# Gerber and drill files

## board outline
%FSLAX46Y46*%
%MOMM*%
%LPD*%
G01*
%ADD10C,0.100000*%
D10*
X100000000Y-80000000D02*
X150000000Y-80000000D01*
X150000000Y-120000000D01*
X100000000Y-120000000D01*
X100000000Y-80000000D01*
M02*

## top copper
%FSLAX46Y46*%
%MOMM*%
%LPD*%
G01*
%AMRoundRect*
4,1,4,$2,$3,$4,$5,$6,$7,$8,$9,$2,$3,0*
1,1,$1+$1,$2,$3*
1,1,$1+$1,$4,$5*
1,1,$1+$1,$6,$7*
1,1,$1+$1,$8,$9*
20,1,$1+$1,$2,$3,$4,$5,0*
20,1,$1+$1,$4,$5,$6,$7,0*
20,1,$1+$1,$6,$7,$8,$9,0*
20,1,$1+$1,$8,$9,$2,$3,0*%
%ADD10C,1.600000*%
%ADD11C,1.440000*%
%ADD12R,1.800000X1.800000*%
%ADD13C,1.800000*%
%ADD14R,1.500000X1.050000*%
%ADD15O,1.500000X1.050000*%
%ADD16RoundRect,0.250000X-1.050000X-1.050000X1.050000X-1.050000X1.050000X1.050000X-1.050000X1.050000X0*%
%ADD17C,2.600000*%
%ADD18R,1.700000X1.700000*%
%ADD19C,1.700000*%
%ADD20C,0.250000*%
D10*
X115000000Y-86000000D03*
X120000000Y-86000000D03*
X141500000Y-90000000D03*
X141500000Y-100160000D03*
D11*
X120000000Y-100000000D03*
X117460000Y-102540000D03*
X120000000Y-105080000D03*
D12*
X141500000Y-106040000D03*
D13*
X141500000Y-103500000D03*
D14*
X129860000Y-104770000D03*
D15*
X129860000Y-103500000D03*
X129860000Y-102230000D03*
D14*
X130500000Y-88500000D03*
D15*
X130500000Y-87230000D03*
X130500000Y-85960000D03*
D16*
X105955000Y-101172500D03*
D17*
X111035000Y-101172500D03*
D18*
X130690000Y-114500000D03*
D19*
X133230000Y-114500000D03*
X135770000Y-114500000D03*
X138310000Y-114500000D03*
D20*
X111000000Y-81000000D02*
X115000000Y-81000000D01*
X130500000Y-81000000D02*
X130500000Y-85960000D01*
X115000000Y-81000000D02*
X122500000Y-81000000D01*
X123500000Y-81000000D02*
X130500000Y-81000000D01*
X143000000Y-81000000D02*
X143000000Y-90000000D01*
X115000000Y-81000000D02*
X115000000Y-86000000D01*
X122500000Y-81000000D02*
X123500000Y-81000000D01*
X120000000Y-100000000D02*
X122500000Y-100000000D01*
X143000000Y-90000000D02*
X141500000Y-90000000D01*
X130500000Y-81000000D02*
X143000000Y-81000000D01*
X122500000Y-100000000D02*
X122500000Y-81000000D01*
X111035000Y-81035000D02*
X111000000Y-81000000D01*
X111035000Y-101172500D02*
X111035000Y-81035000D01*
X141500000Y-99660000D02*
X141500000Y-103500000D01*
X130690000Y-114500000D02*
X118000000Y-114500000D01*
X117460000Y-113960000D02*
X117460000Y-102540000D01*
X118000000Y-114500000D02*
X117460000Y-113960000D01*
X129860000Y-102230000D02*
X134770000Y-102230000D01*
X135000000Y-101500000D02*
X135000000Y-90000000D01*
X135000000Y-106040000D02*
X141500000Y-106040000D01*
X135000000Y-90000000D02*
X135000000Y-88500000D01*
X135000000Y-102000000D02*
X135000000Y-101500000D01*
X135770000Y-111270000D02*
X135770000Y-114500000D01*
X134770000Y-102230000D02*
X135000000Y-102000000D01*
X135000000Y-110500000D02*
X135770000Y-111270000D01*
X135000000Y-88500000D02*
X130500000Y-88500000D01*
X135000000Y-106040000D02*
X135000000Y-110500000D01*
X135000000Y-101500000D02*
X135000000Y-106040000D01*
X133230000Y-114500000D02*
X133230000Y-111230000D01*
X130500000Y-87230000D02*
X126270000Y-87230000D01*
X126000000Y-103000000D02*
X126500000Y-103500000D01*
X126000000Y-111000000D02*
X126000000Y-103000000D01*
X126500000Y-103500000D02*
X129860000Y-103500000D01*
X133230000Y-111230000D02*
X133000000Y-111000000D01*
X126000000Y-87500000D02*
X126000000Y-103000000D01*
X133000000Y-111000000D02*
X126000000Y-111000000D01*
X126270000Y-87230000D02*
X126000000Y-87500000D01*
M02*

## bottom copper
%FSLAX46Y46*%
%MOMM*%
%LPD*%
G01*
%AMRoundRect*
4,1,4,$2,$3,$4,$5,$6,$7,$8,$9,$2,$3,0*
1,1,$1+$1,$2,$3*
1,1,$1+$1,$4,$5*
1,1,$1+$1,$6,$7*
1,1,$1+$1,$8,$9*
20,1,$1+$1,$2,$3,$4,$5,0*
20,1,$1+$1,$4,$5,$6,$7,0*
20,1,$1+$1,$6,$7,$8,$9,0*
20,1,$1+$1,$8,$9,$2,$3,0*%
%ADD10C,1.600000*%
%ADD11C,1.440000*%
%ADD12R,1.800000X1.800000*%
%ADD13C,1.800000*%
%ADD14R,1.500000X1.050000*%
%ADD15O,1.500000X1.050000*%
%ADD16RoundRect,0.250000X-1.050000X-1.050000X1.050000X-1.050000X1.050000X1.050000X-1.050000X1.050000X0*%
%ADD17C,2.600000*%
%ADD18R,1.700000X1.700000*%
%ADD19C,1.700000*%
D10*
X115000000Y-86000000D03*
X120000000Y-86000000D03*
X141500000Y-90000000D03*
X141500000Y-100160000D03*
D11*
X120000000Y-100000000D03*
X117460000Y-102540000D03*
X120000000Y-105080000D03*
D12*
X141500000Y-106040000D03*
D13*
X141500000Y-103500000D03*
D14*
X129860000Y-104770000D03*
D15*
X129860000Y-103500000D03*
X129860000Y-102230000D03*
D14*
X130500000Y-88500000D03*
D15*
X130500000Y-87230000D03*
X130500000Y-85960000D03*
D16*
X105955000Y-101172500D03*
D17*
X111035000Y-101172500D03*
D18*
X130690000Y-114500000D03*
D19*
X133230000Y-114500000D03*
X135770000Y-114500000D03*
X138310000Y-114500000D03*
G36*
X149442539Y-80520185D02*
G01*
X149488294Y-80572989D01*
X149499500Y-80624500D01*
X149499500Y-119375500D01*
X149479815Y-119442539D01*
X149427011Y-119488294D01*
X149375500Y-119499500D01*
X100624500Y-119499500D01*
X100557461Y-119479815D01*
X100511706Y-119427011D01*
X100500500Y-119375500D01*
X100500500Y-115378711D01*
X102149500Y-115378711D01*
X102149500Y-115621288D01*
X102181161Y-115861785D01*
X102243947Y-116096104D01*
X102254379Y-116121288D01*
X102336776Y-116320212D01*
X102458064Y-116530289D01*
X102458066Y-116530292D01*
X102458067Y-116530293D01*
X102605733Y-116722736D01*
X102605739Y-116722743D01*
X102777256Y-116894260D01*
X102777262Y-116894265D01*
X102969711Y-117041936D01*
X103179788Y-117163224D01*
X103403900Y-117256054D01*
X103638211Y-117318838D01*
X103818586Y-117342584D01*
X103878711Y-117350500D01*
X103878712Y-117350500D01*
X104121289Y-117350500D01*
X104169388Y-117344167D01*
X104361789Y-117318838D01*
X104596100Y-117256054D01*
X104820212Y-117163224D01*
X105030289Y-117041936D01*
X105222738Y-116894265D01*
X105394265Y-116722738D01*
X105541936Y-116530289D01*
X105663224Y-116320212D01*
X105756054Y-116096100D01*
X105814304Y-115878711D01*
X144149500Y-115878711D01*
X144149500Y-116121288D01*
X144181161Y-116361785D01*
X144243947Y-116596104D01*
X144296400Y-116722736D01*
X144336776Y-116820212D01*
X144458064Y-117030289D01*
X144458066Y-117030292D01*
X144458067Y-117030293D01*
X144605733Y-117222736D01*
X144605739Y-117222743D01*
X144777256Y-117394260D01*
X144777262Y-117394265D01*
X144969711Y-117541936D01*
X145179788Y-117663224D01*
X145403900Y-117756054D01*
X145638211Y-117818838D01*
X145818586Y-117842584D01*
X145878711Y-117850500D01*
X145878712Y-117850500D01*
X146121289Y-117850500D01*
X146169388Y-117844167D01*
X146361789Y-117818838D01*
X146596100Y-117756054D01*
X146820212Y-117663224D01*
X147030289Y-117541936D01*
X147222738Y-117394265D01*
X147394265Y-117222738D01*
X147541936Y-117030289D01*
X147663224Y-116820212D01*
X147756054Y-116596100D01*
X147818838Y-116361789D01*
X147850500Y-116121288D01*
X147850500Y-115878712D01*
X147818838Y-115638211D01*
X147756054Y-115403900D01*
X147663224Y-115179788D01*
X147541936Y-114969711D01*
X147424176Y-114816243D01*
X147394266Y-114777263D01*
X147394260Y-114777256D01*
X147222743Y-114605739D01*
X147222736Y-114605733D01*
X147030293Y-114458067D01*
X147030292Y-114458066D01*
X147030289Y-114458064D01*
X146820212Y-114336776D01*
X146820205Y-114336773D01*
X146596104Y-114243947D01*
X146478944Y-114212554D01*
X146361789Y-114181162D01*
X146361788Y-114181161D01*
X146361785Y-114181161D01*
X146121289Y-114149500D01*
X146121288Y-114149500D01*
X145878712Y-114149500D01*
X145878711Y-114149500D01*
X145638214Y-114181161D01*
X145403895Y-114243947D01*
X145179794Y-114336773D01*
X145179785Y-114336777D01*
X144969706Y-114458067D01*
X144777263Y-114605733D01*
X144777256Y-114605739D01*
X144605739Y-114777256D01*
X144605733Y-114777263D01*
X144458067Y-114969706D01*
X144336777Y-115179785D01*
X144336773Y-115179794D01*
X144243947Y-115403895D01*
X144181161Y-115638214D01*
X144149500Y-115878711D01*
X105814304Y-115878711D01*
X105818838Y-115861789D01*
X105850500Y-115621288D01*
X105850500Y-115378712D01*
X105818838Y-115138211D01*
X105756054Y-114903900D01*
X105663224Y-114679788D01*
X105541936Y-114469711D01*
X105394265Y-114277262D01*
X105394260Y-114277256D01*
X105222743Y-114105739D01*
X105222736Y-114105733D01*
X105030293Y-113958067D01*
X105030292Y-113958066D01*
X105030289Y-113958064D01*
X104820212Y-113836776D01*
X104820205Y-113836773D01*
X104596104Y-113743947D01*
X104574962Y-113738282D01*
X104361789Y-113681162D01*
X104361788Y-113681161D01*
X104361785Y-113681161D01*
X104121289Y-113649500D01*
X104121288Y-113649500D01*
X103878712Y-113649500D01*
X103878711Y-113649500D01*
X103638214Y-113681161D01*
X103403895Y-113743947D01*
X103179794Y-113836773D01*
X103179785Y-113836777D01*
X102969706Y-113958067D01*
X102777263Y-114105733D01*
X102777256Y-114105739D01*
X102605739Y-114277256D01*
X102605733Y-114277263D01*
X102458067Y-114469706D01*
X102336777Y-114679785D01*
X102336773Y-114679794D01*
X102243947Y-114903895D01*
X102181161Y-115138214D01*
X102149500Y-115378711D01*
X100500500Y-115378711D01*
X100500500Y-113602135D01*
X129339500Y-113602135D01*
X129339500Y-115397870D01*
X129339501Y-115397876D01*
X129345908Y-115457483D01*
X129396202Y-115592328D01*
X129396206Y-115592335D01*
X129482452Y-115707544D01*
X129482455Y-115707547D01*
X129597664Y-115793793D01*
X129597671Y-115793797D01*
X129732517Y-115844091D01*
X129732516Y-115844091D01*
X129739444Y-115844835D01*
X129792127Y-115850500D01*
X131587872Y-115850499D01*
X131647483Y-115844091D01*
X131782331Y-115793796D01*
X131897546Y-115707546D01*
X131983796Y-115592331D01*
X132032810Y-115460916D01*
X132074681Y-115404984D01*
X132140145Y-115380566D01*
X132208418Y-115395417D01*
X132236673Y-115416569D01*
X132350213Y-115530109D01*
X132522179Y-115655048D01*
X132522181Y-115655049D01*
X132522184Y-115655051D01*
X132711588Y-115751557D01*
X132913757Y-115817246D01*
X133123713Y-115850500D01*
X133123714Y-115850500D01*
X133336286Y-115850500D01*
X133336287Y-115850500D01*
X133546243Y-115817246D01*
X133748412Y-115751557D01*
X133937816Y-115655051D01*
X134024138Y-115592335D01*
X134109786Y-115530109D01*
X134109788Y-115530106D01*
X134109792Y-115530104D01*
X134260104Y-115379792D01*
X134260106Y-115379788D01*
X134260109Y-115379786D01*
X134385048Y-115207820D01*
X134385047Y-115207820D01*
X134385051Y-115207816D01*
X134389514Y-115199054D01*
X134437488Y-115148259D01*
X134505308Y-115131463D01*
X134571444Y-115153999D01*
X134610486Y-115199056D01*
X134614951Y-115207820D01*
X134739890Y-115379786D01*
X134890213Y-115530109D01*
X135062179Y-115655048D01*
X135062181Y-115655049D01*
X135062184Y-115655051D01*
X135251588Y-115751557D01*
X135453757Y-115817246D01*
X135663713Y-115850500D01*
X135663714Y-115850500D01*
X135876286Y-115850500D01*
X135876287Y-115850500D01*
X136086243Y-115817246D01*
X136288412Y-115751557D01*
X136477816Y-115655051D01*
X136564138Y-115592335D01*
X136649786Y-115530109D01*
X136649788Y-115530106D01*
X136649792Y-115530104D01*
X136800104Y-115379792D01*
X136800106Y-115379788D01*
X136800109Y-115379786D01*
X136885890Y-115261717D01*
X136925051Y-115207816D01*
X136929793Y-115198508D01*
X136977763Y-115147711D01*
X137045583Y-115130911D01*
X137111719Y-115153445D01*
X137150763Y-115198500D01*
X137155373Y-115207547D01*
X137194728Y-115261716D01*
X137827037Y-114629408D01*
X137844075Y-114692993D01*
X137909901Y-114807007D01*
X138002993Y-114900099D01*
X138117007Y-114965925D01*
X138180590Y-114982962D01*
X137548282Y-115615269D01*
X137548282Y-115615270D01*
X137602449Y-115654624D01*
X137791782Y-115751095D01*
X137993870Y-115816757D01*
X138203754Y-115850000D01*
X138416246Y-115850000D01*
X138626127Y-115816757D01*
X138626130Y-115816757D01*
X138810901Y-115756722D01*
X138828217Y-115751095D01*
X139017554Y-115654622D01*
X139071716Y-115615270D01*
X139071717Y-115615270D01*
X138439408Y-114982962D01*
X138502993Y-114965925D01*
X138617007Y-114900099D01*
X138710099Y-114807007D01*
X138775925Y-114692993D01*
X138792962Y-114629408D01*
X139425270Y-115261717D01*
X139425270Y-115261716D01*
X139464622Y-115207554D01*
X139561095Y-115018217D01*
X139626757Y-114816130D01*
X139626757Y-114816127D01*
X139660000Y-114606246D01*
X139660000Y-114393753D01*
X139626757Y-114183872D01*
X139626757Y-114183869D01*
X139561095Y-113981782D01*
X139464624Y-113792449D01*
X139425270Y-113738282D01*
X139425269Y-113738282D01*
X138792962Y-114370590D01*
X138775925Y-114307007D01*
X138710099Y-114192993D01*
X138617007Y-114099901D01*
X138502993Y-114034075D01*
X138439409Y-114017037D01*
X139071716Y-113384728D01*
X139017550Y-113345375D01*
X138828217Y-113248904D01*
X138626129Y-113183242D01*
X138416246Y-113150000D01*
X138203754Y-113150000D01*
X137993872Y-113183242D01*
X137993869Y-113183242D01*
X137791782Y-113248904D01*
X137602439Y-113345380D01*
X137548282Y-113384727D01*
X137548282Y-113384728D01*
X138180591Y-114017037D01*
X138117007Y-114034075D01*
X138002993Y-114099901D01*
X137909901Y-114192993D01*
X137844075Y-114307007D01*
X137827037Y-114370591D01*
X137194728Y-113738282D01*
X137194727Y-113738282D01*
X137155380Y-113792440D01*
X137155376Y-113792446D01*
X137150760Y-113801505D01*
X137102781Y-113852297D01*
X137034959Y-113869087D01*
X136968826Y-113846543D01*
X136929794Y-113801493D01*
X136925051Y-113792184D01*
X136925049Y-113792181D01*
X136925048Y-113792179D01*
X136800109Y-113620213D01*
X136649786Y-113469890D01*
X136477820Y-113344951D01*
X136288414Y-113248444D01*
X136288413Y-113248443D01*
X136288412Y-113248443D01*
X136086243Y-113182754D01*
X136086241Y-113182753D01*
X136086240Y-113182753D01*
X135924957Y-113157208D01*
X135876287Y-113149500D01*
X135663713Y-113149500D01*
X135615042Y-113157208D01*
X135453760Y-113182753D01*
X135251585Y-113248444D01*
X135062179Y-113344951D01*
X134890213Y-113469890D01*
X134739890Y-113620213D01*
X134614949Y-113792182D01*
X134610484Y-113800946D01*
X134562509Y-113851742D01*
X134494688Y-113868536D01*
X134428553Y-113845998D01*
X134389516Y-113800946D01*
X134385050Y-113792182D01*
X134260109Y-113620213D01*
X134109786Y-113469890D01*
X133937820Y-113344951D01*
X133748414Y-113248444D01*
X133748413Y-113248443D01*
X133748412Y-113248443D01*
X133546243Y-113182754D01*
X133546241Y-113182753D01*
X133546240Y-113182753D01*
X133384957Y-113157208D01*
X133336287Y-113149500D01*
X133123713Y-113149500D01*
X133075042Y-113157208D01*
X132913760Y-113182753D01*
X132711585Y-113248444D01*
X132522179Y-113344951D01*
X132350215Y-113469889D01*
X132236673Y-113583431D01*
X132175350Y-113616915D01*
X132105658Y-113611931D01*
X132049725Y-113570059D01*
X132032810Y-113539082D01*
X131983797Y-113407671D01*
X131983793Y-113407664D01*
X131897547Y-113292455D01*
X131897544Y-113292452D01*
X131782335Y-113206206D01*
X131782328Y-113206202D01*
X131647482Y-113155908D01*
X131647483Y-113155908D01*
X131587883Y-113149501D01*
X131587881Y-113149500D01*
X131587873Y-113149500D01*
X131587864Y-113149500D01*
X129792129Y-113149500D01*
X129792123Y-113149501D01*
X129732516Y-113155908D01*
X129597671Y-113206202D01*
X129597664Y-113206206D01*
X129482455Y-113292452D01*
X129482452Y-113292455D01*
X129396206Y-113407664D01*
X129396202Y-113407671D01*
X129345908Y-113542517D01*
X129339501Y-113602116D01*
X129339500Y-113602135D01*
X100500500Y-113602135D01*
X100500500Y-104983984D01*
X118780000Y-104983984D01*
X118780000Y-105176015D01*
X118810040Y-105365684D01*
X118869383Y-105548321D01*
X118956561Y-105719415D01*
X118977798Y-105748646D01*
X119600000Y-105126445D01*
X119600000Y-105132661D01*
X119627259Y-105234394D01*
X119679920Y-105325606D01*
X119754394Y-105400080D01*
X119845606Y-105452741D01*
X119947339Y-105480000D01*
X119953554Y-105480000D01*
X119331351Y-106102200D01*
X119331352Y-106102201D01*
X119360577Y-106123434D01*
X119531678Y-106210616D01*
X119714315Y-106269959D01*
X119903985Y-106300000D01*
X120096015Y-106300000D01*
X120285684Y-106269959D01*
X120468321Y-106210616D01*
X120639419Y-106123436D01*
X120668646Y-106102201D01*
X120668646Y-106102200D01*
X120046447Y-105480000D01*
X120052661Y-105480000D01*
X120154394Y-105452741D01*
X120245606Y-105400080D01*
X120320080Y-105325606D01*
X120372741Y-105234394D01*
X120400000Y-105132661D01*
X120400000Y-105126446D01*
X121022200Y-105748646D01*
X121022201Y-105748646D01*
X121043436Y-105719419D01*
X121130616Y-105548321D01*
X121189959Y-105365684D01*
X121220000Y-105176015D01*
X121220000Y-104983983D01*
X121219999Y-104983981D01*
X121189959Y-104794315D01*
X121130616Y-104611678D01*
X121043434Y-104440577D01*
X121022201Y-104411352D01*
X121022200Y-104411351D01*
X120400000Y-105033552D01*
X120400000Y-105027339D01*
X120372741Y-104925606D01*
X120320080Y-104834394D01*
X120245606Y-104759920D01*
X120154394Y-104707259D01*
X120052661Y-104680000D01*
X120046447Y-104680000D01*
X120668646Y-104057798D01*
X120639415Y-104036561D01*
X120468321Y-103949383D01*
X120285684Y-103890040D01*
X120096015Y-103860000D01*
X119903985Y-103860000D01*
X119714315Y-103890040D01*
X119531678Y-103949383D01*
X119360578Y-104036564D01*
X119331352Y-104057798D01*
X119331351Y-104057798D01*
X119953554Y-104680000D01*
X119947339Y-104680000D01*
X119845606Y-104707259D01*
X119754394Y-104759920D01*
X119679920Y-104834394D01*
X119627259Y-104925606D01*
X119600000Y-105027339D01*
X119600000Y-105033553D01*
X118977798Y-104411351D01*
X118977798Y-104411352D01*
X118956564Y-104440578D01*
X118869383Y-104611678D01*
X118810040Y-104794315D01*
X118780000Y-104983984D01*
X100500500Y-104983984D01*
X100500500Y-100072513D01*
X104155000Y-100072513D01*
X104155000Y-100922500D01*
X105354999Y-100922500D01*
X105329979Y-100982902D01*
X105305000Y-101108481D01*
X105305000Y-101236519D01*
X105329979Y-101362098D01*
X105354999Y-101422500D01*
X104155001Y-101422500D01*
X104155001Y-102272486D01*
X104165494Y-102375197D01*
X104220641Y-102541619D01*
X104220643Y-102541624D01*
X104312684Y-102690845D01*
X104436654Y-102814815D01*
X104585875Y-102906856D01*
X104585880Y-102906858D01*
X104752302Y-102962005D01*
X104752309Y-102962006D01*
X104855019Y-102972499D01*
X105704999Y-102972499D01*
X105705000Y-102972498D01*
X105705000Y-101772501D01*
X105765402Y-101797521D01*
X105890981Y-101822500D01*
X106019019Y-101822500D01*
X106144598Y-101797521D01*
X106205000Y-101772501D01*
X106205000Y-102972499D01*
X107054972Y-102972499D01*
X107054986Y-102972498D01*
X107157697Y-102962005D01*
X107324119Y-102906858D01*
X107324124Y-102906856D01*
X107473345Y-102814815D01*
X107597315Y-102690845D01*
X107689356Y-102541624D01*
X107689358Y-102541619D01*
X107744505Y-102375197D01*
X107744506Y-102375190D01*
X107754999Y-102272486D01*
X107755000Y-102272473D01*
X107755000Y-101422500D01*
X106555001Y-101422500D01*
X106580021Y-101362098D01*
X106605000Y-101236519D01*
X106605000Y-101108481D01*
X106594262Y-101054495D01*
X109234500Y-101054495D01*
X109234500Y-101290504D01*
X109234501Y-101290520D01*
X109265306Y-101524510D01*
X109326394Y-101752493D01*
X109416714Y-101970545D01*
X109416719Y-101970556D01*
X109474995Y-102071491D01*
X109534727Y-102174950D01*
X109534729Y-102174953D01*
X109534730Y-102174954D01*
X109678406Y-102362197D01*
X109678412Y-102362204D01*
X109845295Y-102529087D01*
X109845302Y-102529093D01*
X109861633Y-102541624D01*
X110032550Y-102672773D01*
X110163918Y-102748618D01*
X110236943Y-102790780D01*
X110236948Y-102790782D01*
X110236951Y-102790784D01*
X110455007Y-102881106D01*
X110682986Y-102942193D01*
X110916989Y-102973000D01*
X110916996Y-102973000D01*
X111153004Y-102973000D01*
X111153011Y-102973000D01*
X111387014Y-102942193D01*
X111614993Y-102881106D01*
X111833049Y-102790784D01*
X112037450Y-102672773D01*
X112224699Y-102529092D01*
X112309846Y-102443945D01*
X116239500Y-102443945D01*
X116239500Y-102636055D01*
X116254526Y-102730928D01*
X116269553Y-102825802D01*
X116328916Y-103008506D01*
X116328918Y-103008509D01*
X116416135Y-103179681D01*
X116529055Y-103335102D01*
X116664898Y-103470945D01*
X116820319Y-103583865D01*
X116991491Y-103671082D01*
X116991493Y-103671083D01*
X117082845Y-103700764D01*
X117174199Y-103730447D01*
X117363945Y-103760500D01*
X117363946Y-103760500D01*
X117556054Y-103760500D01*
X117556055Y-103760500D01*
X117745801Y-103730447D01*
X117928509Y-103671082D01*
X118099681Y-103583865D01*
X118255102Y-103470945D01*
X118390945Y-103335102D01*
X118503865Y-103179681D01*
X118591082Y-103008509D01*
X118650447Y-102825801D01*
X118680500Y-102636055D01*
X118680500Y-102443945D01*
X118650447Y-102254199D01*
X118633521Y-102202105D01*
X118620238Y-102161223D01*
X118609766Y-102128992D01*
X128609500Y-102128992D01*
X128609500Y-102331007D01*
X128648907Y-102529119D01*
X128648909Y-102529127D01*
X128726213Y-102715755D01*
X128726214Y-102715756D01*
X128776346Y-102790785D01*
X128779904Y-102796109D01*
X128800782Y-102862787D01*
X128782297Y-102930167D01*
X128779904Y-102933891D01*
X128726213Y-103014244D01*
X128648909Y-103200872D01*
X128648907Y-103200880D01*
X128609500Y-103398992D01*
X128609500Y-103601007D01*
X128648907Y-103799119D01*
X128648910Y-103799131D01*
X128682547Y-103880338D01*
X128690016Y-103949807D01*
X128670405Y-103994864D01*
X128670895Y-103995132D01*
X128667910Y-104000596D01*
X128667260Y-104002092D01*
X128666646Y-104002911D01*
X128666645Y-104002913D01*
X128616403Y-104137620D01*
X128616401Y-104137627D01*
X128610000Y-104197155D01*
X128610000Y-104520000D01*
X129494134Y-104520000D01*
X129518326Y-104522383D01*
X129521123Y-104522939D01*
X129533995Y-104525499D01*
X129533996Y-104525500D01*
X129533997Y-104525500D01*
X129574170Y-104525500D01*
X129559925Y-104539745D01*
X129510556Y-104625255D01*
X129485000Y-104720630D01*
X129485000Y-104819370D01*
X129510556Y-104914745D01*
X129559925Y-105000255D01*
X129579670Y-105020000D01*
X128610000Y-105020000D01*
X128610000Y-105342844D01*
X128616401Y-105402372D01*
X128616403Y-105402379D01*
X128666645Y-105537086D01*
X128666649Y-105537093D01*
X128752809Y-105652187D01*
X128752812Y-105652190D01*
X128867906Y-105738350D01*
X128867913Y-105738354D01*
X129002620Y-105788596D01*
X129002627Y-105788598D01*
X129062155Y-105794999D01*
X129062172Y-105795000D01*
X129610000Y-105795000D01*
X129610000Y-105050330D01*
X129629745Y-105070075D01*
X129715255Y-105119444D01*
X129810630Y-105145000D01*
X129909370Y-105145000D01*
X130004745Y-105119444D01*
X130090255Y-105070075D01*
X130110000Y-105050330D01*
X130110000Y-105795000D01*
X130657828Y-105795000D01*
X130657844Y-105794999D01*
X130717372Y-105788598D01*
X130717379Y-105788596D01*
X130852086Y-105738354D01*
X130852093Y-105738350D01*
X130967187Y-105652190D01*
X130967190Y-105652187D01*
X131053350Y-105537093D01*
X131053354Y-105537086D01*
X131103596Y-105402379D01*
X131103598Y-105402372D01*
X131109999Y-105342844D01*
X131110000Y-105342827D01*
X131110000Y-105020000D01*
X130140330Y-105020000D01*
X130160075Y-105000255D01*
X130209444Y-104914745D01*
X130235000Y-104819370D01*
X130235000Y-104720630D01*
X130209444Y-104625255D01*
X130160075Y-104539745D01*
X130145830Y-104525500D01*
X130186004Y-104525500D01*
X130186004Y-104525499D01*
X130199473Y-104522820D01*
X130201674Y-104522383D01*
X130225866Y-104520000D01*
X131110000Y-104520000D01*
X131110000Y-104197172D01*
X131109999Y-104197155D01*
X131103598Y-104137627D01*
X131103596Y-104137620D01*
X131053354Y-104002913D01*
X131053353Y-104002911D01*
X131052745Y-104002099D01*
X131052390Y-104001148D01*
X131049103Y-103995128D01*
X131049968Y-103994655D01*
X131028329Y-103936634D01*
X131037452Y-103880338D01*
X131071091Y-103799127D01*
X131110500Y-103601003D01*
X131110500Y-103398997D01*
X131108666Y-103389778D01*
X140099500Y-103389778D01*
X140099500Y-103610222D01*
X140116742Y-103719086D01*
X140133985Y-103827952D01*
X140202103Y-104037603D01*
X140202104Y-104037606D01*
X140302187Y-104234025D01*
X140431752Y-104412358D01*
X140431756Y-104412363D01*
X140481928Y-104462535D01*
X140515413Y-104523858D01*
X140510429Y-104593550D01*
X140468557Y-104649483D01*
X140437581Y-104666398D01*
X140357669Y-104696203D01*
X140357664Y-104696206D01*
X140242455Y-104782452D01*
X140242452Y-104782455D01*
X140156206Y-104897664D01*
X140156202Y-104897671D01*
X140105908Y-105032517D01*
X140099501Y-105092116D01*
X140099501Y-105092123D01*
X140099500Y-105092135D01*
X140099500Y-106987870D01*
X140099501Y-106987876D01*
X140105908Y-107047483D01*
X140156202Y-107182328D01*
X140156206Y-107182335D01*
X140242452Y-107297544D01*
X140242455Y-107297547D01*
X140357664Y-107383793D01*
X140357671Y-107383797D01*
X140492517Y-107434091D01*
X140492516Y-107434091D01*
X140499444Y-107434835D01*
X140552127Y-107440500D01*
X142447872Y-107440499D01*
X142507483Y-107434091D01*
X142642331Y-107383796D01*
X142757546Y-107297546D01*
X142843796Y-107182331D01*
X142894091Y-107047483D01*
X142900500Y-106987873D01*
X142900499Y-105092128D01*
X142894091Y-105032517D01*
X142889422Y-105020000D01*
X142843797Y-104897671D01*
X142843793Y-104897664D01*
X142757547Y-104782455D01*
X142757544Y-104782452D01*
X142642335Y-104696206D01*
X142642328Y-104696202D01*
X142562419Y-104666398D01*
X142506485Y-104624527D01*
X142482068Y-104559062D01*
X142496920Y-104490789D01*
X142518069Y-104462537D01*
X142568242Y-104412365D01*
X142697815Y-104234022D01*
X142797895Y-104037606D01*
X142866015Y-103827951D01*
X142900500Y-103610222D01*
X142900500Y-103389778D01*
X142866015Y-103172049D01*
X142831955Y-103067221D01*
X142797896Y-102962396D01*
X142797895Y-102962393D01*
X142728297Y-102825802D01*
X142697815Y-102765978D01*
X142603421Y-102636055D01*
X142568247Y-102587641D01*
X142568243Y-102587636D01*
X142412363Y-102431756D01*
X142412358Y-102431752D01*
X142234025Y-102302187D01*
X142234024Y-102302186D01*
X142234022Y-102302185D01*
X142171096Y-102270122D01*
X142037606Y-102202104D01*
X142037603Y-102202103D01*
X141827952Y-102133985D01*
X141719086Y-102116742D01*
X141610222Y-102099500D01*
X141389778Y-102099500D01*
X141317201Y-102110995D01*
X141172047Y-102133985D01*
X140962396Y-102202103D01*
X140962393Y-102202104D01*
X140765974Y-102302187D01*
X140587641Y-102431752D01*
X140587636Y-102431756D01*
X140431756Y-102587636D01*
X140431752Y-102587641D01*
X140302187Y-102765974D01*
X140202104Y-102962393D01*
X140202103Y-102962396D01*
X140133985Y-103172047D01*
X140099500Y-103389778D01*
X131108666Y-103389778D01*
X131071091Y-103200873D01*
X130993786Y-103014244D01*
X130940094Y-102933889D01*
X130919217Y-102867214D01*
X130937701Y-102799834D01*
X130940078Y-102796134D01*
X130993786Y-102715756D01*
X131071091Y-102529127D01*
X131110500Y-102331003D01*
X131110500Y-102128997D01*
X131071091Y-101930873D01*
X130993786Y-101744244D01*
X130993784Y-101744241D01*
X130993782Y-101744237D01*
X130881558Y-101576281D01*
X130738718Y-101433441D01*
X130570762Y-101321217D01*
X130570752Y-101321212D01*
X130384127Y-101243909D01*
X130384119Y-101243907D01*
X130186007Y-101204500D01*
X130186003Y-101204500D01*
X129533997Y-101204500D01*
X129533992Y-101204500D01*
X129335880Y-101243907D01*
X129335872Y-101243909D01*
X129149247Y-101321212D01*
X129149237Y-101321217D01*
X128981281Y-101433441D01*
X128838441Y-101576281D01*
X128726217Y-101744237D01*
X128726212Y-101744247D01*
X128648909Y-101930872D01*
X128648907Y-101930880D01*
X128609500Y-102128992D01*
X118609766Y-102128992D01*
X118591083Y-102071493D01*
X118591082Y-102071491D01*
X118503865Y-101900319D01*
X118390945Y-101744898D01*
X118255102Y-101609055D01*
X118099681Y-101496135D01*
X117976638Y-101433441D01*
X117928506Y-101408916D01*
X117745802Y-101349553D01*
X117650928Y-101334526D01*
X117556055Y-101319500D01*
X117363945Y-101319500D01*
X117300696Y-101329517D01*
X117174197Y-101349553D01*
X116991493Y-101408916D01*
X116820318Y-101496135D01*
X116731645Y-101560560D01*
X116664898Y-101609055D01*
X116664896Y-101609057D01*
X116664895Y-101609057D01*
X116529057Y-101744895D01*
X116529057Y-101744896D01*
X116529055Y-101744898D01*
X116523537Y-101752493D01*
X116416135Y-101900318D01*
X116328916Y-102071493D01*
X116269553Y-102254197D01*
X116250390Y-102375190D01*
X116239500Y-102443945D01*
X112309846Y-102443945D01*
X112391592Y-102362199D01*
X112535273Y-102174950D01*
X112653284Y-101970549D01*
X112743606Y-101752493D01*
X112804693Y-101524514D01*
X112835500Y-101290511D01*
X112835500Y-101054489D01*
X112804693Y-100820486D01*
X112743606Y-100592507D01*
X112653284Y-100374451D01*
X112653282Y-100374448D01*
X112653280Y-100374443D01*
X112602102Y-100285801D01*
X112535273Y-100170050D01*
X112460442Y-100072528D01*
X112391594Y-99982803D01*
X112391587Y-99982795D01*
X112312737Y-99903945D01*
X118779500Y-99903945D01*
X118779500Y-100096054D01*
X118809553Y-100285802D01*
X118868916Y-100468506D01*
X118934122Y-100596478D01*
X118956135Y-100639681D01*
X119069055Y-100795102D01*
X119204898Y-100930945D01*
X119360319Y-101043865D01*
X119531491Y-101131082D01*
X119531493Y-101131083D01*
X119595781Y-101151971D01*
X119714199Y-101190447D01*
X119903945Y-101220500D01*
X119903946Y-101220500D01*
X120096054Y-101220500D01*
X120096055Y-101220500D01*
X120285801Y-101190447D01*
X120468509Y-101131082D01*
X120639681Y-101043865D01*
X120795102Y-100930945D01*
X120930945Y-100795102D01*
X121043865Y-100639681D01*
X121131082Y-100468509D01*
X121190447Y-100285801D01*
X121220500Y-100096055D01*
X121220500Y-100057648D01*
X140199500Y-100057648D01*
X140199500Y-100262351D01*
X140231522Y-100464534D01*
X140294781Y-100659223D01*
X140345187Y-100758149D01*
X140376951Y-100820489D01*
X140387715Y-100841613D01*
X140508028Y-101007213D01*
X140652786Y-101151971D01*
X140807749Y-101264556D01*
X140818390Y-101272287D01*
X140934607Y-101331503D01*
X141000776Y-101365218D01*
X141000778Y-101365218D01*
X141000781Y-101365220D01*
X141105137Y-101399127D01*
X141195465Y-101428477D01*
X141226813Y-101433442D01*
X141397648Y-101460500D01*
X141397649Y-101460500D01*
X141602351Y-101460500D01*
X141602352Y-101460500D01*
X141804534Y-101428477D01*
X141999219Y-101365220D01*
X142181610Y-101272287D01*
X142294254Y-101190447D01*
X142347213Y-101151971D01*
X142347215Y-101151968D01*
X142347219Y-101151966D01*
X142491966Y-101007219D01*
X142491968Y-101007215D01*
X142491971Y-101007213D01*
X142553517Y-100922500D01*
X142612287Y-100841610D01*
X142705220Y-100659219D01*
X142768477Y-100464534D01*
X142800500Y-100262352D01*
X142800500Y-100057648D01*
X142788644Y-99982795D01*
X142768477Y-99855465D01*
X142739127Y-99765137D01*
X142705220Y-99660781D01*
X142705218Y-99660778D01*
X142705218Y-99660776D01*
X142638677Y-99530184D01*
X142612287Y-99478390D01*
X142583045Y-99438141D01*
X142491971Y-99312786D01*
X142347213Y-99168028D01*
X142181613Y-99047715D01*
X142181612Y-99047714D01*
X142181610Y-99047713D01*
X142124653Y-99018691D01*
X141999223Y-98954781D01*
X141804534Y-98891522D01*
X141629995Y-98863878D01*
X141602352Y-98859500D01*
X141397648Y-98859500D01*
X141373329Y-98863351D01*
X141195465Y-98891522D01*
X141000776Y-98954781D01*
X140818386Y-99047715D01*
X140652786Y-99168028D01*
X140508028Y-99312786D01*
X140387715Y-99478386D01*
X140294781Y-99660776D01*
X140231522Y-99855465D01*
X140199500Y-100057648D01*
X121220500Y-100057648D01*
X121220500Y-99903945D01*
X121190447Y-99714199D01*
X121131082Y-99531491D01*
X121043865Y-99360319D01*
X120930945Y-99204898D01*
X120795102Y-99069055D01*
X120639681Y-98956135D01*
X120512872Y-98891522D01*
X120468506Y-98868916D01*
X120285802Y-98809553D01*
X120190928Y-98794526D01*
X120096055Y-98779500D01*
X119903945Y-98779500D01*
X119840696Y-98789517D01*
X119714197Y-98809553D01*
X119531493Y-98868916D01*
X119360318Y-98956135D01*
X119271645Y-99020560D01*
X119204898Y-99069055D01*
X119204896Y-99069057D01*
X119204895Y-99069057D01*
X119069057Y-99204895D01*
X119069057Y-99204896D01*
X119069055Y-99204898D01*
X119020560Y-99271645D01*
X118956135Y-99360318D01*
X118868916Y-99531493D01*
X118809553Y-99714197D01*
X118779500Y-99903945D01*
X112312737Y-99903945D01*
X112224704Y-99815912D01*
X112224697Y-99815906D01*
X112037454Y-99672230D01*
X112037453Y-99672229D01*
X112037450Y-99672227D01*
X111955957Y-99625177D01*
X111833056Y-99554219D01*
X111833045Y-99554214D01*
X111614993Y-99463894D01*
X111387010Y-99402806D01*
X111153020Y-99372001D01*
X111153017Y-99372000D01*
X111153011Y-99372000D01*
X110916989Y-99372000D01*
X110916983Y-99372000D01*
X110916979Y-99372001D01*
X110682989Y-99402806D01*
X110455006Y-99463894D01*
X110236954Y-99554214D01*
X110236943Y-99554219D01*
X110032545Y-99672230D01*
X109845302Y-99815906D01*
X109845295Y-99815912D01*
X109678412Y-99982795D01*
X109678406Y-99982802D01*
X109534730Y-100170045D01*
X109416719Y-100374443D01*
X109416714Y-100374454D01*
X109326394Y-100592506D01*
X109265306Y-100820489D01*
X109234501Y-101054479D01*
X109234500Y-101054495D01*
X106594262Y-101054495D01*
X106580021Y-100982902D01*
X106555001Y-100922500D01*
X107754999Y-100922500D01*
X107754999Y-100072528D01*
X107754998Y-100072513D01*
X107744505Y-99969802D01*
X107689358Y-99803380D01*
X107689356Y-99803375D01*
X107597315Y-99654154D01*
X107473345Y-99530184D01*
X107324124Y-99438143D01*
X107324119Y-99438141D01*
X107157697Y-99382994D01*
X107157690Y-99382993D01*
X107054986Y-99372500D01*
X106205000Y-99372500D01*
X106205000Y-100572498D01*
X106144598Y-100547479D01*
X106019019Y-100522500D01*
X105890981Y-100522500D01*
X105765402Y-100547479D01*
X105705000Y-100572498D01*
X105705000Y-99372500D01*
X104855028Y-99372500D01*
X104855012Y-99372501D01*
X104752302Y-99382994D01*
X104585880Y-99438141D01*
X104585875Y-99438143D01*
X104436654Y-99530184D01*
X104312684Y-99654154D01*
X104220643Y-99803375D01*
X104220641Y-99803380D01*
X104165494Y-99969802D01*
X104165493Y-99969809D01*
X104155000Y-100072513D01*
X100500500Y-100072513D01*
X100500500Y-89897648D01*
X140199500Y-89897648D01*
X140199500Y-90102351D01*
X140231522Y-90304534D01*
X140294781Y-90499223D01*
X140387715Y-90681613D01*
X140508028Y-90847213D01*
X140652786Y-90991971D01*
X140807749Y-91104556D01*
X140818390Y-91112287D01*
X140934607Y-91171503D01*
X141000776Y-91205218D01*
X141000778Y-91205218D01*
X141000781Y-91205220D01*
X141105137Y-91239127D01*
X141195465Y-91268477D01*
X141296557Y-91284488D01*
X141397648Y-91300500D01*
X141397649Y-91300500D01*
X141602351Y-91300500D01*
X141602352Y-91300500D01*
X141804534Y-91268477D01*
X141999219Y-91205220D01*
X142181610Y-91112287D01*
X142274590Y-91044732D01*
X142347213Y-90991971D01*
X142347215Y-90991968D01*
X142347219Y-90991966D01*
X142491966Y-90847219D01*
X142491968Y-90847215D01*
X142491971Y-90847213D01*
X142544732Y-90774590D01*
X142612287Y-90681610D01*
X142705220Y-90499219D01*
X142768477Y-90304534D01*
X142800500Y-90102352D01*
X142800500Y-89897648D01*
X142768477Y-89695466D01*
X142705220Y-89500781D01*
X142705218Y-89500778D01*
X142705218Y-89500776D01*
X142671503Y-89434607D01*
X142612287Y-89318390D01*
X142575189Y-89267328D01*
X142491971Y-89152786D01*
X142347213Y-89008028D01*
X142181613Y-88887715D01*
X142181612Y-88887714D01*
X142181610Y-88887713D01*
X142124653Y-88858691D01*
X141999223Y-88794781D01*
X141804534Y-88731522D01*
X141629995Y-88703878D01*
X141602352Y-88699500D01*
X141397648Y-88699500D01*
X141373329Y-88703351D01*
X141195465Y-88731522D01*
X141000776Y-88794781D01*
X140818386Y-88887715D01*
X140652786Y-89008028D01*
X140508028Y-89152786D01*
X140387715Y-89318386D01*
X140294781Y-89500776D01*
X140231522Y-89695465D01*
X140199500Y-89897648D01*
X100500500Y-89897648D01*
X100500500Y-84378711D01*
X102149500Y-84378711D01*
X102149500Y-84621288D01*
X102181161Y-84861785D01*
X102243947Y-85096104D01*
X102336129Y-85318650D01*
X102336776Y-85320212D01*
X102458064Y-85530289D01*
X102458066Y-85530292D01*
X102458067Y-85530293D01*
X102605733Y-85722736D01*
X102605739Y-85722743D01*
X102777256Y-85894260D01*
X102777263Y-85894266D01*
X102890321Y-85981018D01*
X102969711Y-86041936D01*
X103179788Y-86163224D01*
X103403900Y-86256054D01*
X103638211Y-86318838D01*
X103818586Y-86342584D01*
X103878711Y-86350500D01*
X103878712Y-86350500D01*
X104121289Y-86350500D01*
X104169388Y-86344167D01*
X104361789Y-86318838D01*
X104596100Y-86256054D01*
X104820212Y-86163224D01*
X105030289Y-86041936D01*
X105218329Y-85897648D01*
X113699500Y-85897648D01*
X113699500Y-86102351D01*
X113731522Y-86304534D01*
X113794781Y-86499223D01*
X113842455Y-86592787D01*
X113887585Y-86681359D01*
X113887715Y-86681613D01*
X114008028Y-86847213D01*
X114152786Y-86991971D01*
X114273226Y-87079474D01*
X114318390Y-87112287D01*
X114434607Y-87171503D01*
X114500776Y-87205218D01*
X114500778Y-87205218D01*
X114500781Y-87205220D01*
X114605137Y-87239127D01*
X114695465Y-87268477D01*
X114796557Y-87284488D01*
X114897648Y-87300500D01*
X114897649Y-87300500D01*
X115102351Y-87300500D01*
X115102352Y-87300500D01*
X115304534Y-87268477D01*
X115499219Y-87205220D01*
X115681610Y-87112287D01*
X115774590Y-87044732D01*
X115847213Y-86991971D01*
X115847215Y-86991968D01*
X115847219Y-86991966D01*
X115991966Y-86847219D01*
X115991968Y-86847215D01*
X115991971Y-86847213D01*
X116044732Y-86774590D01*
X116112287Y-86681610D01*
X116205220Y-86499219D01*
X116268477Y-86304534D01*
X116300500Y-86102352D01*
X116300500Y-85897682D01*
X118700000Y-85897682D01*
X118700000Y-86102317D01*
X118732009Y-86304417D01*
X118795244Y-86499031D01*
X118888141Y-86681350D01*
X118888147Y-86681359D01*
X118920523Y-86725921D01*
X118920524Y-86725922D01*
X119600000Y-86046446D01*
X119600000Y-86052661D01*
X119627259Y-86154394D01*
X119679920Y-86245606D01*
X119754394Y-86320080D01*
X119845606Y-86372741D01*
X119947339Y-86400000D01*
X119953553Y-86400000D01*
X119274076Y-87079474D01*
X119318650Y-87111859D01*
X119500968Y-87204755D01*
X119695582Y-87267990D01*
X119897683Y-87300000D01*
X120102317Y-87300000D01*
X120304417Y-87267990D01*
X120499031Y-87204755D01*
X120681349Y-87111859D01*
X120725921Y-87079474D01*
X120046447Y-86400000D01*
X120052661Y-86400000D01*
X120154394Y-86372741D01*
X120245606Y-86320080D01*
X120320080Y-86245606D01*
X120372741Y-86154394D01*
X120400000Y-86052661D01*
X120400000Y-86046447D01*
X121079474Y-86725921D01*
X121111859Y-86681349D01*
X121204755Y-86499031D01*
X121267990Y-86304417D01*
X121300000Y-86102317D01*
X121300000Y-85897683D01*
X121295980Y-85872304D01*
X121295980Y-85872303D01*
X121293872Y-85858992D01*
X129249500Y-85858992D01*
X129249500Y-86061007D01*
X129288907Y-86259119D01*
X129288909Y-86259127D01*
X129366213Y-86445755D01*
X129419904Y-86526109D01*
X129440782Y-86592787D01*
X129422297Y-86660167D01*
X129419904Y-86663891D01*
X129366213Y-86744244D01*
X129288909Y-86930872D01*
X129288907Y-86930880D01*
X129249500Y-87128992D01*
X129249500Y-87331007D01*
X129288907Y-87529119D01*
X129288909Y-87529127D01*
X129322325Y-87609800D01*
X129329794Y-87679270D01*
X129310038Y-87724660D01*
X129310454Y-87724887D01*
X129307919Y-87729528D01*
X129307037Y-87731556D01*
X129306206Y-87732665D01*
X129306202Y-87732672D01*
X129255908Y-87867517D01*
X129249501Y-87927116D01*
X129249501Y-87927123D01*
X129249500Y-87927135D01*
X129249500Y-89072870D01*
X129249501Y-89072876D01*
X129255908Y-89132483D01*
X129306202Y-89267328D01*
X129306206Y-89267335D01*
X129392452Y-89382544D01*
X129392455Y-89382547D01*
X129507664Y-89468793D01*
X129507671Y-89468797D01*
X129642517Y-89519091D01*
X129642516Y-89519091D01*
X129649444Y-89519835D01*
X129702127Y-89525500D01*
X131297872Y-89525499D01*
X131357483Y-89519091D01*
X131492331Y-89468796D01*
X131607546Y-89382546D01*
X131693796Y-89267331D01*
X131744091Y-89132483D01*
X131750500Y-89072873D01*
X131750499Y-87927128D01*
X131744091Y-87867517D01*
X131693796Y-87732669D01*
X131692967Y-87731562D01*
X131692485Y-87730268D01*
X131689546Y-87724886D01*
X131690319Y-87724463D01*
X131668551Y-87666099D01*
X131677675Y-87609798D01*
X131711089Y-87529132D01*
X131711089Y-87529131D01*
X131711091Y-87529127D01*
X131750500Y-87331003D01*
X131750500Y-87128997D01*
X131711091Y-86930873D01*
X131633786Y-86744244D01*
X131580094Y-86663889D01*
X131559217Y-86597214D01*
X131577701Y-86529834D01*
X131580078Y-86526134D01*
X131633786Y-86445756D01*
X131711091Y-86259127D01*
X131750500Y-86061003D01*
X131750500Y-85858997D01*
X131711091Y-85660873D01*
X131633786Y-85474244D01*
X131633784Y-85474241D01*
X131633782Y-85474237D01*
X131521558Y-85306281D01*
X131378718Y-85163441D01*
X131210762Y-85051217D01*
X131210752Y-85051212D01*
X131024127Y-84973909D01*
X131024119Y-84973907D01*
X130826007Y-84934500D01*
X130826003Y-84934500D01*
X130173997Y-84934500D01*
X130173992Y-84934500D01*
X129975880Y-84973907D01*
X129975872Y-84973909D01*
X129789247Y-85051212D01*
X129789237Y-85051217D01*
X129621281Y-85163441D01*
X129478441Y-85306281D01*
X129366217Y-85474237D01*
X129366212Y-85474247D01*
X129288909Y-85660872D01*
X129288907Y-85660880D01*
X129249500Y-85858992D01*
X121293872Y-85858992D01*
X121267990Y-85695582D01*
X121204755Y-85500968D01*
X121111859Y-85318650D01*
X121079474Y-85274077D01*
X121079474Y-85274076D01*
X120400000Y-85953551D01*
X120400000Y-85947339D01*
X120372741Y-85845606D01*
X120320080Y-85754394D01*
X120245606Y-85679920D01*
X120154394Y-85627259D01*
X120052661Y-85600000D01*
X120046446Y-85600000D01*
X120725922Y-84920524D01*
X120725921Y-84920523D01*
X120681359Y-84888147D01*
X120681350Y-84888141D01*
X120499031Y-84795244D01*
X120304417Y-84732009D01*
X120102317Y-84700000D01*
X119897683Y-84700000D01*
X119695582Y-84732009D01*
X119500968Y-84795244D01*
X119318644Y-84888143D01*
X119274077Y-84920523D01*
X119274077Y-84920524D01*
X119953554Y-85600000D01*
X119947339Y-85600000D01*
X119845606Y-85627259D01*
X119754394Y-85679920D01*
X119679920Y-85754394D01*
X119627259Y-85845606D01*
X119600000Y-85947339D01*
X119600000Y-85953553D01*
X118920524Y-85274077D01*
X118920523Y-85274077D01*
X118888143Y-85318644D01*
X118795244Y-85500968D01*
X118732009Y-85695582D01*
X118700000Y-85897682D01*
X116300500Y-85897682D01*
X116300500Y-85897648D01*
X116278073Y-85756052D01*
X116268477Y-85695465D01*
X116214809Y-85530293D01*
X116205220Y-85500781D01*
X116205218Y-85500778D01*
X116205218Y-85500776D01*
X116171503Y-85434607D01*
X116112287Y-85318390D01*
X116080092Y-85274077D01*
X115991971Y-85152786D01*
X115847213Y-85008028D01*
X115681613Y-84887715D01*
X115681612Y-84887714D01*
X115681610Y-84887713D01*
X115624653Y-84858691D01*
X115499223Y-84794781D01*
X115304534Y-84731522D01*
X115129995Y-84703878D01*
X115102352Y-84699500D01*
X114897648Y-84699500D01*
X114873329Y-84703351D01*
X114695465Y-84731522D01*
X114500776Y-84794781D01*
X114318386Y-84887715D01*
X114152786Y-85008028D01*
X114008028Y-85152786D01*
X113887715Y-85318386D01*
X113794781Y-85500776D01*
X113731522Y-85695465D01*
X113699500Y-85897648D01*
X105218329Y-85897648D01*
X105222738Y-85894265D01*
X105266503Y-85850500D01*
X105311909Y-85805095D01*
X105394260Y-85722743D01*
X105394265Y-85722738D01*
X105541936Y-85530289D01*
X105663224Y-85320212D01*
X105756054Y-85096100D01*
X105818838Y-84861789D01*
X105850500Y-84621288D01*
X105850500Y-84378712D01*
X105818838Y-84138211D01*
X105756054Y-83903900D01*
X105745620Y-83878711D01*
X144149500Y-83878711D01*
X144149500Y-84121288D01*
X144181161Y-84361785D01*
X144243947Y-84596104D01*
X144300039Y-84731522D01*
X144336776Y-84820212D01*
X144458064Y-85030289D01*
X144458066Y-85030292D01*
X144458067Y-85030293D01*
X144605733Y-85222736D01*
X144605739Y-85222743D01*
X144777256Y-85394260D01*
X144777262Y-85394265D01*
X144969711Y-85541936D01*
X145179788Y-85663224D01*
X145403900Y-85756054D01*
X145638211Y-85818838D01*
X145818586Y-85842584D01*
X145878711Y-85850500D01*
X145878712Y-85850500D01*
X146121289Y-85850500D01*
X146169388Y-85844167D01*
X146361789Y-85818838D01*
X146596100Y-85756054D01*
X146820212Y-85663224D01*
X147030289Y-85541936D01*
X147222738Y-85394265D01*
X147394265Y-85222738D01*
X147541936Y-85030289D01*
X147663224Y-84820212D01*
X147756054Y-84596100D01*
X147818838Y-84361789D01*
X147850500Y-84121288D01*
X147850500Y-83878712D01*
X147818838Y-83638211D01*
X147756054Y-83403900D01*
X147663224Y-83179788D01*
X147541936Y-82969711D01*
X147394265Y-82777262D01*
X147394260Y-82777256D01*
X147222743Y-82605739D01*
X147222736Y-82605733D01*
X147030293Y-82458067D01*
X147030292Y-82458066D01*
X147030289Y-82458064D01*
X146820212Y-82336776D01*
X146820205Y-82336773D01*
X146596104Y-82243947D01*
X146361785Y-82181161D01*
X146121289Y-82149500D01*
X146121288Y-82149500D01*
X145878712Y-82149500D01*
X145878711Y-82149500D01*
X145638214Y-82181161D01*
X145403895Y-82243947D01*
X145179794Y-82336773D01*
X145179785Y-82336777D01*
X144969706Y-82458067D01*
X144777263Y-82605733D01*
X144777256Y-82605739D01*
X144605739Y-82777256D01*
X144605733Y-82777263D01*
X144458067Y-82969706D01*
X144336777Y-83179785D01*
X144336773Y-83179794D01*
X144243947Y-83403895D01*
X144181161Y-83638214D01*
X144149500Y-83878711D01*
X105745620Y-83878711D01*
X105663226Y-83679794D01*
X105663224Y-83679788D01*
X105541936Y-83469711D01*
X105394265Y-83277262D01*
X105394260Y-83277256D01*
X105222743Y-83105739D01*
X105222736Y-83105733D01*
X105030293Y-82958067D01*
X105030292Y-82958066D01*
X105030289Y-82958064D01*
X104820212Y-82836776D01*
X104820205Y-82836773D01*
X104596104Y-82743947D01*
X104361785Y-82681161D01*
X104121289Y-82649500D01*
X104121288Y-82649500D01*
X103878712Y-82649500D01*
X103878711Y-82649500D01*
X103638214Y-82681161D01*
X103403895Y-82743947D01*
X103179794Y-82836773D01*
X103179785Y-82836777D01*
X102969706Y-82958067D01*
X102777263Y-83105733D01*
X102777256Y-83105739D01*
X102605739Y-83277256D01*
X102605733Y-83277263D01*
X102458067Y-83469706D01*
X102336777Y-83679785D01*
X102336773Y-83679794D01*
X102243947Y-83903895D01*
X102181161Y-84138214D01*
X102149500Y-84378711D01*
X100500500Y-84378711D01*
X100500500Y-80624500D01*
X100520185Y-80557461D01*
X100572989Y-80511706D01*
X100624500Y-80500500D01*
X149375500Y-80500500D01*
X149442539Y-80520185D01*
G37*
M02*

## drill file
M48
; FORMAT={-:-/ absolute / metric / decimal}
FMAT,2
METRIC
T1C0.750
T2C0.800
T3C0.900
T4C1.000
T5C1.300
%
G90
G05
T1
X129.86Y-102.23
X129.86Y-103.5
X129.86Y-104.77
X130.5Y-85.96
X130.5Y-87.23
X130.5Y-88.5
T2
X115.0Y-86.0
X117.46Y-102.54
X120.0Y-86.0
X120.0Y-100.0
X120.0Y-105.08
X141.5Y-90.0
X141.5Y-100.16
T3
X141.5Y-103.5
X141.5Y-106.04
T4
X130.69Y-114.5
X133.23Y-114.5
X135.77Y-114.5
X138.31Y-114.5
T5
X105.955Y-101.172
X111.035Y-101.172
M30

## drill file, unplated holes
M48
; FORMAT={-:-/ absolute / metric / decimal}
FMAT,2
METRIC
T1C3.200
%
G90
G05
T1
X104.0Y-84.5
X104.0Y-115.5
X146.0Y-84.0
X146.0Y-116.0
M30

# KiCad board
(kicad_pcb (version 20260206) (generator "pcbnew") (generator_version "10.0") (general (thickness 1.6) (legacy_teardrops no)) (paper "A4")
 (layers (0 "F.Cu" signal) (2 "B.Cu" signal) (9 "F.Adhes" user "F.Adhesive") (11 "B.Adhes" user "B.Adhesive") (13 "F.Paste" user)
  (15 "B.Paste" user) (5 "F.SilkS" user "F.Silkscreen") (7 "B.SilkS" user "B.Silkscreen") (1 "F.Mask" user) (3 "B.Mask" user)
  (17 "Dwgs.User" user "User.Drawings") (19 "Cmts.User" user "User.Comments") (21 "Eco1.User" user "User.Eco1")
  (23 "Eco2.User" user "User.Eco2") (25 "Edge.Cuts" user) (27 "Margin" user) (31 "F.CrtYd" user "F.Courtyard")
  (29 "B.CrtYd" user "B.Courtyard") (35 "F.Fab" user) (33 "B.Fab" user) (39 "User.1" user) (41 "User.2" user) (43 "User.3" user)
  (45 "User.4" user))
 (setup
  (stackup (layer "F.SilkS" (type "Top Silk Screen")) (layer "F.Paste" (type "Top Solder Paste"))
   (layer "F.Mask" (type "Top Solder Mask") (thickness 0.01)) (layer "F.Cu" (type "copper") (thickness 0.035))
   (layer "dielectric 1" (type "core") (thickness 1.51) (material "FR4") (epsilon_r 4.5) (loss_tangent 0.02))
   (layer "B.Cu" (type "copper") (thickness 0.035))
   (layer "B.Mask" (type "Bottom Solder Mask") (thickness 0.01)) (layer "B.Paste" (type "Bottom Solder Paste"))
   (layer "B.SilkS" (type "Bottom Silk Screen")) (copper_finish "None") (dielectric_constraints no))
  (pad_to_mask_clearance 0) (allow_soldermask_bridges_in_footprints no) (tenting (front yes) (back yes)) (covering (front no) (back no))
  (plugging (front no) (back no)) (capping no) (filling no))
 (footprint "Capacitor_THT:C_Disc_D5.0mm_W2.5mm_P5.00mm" (layer "F.Cu") (at 115 86)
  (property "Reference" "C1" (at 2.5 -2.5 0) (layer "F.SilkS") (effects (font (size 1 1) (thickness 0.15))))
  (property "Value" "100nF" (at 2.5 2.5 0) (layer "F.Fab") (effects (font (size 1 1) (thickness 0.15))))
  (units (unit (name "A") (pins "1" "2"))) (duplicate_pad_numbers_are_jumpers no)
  (pad "1" thru_hole circle (at 0 0) (size 1.6 1.6) (drill 0.8) (layers "*.Cu" "*.Mask") (remove_unused_layers no) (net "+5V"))
  (pad "2" thru_hole circle (at 5 0) (size 1.6 1.6) (drill 0.8) (layers "*.Cu" "*.Mask") (remove_unused_layers no) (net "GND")))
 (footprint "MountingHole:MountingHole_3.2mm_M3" (layer "F.Cu") (at 104 115.5)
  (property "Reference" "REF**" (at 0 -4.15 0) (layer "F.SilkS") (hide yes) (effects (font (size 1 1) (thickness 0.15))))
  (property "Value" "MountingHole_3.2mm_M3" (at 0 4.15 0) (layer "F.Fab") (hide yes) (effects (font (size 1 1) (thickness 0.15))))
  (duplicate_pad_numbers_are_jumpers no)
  (pad "" np_thru_hole circle (at 0 0) (size 3.2 3.2) (drill 3.2) (layers "*.Cu" "*.Mask")))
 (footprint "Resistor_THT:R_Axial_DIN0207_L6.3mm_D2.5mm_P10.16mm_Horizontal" (layer "F.Cu") (at 141.5 90 -90)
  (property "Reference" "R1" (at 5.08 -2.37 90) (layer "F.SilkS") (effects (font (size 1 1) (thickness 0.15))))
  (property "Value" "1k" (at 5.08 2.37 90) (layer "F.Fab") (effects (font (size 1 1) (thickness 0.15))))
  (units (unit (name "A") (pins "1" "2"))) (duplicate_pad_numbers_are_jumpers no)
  (pad "1" thru_hole circle (at 0 0 270) (size 1.6 1.6) (drill 0.8) (layers "*.Cu" "*.Mask") (remove_unused_layers no) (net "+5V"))
  (pad "2" thru_hole circle (at 10.16 0 270) (size 1.6 1.6) (drill 0.8) (layers "*.Cu" "*.Mask") (remove_unused_layers no)
   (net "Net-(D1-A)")))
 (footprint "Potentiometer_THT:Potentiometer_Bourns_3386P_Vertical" (layer "F.Cu") (at 120 100 180)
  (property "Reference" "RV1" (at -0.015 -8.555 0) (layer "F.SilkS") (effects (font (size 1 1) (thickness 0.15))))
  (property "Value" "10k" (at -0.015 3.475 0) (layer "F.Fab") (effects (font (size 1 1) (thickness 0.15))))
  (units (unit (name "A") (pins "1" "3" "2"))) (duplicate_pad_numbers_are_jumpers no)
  (pad "1" thru_hole circle (at 0 0 180) (size 1.44 1.44) (drill 0.8) (layers "*.Cu" "*.Mask") (remove_unused_layers no) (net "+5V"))
  (pad "2" thru_hole circle (at 2.54 -2.54 180) (size 1.44 1.44) (drill 0.8) (layers "*.Cu" "*.Mask") (remove_unused_layers no)
   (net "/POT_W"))
  (pad "3" thru_hole circle (at 0 -5.08 180) (size 1.44 1.44) (drill 0.8) (layers "*.Cu" "*.Mask") (remove_unused_layers no) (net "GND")))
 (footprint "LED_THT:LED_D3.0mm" (layer "F.Cu") (at 141.5 106.04 90)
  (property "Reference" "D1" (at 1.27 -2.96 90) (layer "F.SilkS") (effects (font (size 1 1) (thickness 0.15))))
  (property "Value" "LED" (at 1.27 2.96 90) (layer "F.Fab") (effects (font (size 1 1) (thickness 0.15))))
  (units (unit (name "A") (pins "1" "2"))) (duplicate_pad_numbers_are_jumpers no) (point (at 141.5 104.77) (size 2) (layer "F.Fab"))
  (pad "1" thru_hole rect (at 0 0 90) (size 1.8 1.8) (drill 0.9) (layers "*.Cu" "*.Mask") (remove_unused_layers no) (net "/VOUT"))
  (pad "2" thru_hole circle (at 2.54 0 90) (size 1.8 1.8) (drill 0.9) (layers "*.Cu" "*.Mask") (remove_unused_layers no) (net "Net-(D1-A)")))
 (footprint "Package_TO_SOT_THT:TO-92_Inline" (layer "F.Cu") (at 129.86 104.77 90)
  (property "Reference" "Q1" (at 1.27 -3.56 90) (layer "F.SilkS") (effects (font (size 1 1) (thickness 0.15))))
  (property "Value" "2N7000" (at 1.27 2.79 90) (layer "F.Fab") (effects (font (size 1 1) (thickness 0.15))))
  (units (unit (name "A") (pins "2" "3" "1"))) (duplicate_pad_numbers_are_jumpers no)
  (pad "1" thru_hole rect (at 0 0 90) (size 1.05 1.5) (drill 0.75) (layers "*.Cu" "*.Mask") (remove_unused_layers no) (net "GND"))
  (pad "2" thru_hole oval (at 1.27 0 90) (size 1.05 1.5) (drill 0.75) (layers "*.Cu" "*.Mask") (remove_unused_layers no) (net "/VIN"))
  (pad "3" thru_hole oval (at 2.54 0 90) (size 1.05 1.5) (drill 0.75) (layers "*.Cu" "*.Mask") (remove_unused_layers no) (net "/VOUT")))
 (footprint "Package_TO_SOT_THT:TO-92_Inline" (layer "F.Cu") (at 130.5 88.5 90)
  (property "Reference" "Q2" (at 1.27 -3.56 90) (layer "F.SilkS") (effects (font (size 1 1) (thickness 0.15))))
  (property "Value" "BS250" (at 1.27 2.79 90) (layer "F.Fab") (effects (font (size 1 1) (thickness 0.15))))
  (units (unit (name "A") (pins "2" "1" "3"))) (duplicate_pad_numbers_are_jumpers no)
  (pad "1" thru_hole rect (at 0 0 90) (size 1.05 1.5) (drill 0.75) (layers "*.Cu" "*.Mask") (remove_unused_layers no) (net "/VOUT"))
  (pad "2" thru_hole oval (at 1.27 0 90) (size 1.05 1.5) (drill 0.75) (layers "*.Cu" "*.Mask") (remove_unused_layers no) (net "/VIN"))
  (pad "3" thru_hole oval (at 2.54 0 90) (size 1.05 1.5) (drill 0.75) (layers "*.Cu" "*.Mask") (remove_unused_layers no) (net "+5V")))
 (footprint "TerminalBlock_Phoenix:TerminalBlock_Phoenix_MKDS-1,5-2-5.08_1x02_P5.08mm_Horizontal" (layer "F.Cu") (at 105.955 101.1725)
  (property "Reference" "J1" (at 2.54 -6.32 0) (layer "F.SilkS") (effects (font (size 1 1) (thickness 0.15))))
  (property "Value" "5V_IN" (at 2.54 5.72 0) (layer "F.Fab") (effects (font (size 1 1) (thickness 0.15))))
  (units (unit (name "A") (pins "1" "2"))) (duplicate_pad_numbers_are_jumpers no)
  (pad "1" thru_hole roundrect (at 0 0) (size 2.6 2.6) (drill 1.3) (layers "*.Cu" "*.Mask") (remove_unused_layers no)
   (roundrect_rratio 0.096154) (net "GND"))
  (pad "2" thru_hole circle (at 5.08 0) (size 2.6 2.6) (drill 1.3) (layers "*.Cu" "*.Mask") (remove_unused_layers no) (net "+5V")))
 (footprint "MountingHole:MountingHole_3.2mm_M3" (layer "F.Cu") (at 146 84)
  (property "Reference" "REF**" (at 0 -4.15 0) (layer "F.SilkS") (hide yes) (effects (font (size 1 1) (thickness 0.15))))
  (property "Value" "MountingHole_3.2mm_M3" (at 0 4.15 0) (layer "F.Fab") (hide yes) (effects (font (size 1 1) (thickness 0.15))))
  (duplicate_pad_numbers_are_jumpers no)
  (pad "" np_thru_hole circle (at 0 0) (size 3.2 3.2) (drill 3.2) (layers "*.Cu" "*.Mask")))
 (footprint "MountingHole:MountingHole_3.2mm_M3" (layer "F.Cu") (at 146 116)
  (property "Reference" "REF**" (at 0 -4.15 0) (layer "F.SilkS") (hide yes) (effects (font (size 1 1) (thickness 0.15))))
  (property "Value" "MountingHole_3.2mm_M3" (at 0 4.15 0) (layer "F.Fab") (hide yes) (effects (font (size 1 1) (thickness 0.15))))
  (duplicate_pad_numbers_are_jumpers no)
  (pad "" np_thru_hole circle (at 0 0) (size 3.2 3.2) (drill 3.2) (layers "*.Cu" "*.Mask")))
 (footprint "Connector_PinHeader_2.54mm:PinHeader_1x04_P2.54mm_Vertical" (layer "F.Cu") (at 130.69 114.5 90)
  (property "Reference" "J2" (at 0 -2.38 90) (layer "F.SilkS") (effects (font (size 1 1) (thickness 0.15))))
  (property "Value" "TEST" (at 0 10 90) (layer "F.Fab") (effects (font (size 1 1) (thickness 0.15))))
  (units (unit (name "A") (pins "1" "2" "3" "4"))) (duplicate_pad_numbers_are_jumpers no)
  (pad "1" thru_hole rect (at 0 0 90) (size 1.7 1.7) (drill 1) (layers "*.Cu" "*.Mask") (remove_unused_layers no) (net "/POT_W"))
  (pad "2" thru_hole circle (at 0 2.54 90) (size 1.7 1.7) (drill 1) (layers "*.Cu" "*.Mask") (remove_unused_layers no) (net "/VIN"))
  (pad "3" thru_hole circle (at 0 5.08 90) (size 1.7 1.7) (drill 1) (layers "*.Cu" "*.Mask") (remove_unused_layers no) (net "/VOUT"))
  (pad "4" thru_hole circle (at 0 7.62 90) (size 1.7 1.7) (drill 1) (layers "*.Cu" "*.Mask") (remove_unused_layers no) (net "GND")))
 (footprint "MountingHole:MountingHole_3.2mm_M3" (layer "F.Cu") (at 104 84.5)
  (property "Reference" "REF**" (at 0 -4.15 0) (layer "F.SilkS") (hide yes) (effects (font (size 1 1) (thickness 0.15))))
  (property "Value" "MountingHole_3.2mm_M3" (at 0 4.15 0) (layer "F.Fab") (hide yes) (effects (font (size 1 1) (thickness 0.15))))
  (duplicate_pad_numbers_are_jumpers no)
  (pad "" np_thru_hole circle (at 0 0) (size 3.2 3.2) (drill 3.2) (layers "*.Cu" "*.Mask")))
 (gr_rect (start 100 80) (end 150 120) (stroke (width 0.1) (type default)) (fill no) (layer "Edge.Cuts"))
 (segment (start 111 81) (end 115 81) (width 0.25) (layer "F.Cu") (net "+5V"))
 (segment (start 130.5 81) (end 130.5 85.96) (width 0.25) (layer "F.Cu") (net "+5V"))
 (segment (start 115 81) (end 122.5 81) (width 0.25) (layer "F.Cu") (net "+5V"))
 (segment (start 123.5 81) (end 130.5 81) (width 0.25) (layer "F.Cu") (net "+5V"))
 (segment (start 143 81) (end 143 90) (width 0.25) (layer "F.Cu") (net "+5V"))
 (segment (start 115 81) (end 115 86) (width 0.25) (layer "F.Cu") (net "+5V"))
 (segment (start 122.5 81) (end 123.5 81) (width 0.25) (layer "F.Cu") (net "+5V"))
 (segment (start 120 100) (end 122.5 100) (width 0.25) (layer "F.Cu") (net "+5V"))
 (segment (start 143 90) (end 141.5 90) (width 0.25) (layer "F.Cu") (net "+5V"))
 (segment (start 130.5 81) (end 143 81) (width 0.25) (layer "F.Cu") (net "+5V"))
 (segment (start 122.5 100) (end 122.5 81) (width 0.25) (layer "F.Cu") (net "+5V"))
 (segment (start 111.035 81.035) (end 111 81) (width 0.25) (layer "F.Cu") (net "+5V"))
 (segment (start 111.035 101.1725) (end 111.035 81.035) (width 0.25) (layer "F.Cu") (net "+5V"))
 (segment (start 141.5 99.66) (end 141.5 103.5) (width 0.25) (layer "F.Cu") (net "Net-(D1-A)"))
 (segment (start 130.69 114.5) (end 118 114.5) (width 0.25) (layer "F.Cu") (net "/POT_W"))
 (segment (start 117.46 113.96) (end 117.46 102.54) (width 0.25) (layer "F.Cu") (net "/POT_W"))
 (segment (start 118 114.5) (end 117.46 113.96) (width 0.25) (layer "F.Cu") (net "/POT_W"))
 (segment (start 129.86 102.23) (end 134.77 102.23) (width 0.25) (layer "F.Cu") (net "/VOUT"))
 (segment (start 135 101.5) (end 135 90) (width 0.25) (layer "F.Cu") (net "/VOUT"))
 (segment (start 135 106.04) (end 141.5 106.04) (width 0.25) (layer "F.Cu") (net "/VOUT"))
 (segment (start 135 90) (end 135 88.5) (width 0.25) (layer "F.Cu") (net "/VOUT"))
 (segment (start 135 102) (end 135 101.5) (width 0.25) (layer "F.Cu") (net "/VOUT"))
 (segment (start 135.77 111.27) (end 135.77 114.5) (width 0.25) (layer "F.Cu") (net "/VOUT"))
 (segment (start 134.77 102.23) (end 135 102) (width 0.25) (layer "F.Cu") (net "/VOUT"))
 (segment (start 135 110.5) (end 135.77 111.27) (width 0.25) (layer "F.Cu") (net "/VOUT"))
 (segment (start 135 88.5) (end 130.5 88.5) (width 0.25) (layer "F.Cu") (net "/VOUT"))
 (segment (start 135 106.04) (end 135 110.5) (width 0.25) (layer "F.Cu") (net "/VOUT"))
 (segment (start 135 101.5) (end 135 106.04) (width 0.25) (layer "F.Cu") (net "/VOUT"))
 (segment (start 133.23 114.5) (end 133.23 111.23) (width 0.25) (layer "F.Cu") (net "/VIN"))
 (segment (start 130.5 87.23) (end 126.27 87.23) (width 0.25) (layer "F.Cu") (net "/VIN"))
 (segment (start 126 103) (end 126.5 103.5) (width 0.25) (layer "F.Cu") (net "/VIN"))
 (segment (start 126 111) (end 126 103) (width 0.25) (layer "F.Cu") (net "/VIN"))
 (segment (start 126.5 103.5) (end 129.86 103.5) (width 0.25) (layer "F.Cu") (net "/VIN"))
 (segment (start 133.23 111.23) (end 133 111) (width 0.25) (layer "F.Cu") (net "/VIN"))
 (segment (start 126 87.5) (end 126 103) (width 0.25) (layer "F.Cu") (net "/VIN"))
 (segment (start 133 111) (end 126 111) (width 0.25) (layer "F.Cu") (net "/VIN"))
 (segment (start 126.27 87.23) (end 126 87.5) (width 0.25) (layer "F.Cu") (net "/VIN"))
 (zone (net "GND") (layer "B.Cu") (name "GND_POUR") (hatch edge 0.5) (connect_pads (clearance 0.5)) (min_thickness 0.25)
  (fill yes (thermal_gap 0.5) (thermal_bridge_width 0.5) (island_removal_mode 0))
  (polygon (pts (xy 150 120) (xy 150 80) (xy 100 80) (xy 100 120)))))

